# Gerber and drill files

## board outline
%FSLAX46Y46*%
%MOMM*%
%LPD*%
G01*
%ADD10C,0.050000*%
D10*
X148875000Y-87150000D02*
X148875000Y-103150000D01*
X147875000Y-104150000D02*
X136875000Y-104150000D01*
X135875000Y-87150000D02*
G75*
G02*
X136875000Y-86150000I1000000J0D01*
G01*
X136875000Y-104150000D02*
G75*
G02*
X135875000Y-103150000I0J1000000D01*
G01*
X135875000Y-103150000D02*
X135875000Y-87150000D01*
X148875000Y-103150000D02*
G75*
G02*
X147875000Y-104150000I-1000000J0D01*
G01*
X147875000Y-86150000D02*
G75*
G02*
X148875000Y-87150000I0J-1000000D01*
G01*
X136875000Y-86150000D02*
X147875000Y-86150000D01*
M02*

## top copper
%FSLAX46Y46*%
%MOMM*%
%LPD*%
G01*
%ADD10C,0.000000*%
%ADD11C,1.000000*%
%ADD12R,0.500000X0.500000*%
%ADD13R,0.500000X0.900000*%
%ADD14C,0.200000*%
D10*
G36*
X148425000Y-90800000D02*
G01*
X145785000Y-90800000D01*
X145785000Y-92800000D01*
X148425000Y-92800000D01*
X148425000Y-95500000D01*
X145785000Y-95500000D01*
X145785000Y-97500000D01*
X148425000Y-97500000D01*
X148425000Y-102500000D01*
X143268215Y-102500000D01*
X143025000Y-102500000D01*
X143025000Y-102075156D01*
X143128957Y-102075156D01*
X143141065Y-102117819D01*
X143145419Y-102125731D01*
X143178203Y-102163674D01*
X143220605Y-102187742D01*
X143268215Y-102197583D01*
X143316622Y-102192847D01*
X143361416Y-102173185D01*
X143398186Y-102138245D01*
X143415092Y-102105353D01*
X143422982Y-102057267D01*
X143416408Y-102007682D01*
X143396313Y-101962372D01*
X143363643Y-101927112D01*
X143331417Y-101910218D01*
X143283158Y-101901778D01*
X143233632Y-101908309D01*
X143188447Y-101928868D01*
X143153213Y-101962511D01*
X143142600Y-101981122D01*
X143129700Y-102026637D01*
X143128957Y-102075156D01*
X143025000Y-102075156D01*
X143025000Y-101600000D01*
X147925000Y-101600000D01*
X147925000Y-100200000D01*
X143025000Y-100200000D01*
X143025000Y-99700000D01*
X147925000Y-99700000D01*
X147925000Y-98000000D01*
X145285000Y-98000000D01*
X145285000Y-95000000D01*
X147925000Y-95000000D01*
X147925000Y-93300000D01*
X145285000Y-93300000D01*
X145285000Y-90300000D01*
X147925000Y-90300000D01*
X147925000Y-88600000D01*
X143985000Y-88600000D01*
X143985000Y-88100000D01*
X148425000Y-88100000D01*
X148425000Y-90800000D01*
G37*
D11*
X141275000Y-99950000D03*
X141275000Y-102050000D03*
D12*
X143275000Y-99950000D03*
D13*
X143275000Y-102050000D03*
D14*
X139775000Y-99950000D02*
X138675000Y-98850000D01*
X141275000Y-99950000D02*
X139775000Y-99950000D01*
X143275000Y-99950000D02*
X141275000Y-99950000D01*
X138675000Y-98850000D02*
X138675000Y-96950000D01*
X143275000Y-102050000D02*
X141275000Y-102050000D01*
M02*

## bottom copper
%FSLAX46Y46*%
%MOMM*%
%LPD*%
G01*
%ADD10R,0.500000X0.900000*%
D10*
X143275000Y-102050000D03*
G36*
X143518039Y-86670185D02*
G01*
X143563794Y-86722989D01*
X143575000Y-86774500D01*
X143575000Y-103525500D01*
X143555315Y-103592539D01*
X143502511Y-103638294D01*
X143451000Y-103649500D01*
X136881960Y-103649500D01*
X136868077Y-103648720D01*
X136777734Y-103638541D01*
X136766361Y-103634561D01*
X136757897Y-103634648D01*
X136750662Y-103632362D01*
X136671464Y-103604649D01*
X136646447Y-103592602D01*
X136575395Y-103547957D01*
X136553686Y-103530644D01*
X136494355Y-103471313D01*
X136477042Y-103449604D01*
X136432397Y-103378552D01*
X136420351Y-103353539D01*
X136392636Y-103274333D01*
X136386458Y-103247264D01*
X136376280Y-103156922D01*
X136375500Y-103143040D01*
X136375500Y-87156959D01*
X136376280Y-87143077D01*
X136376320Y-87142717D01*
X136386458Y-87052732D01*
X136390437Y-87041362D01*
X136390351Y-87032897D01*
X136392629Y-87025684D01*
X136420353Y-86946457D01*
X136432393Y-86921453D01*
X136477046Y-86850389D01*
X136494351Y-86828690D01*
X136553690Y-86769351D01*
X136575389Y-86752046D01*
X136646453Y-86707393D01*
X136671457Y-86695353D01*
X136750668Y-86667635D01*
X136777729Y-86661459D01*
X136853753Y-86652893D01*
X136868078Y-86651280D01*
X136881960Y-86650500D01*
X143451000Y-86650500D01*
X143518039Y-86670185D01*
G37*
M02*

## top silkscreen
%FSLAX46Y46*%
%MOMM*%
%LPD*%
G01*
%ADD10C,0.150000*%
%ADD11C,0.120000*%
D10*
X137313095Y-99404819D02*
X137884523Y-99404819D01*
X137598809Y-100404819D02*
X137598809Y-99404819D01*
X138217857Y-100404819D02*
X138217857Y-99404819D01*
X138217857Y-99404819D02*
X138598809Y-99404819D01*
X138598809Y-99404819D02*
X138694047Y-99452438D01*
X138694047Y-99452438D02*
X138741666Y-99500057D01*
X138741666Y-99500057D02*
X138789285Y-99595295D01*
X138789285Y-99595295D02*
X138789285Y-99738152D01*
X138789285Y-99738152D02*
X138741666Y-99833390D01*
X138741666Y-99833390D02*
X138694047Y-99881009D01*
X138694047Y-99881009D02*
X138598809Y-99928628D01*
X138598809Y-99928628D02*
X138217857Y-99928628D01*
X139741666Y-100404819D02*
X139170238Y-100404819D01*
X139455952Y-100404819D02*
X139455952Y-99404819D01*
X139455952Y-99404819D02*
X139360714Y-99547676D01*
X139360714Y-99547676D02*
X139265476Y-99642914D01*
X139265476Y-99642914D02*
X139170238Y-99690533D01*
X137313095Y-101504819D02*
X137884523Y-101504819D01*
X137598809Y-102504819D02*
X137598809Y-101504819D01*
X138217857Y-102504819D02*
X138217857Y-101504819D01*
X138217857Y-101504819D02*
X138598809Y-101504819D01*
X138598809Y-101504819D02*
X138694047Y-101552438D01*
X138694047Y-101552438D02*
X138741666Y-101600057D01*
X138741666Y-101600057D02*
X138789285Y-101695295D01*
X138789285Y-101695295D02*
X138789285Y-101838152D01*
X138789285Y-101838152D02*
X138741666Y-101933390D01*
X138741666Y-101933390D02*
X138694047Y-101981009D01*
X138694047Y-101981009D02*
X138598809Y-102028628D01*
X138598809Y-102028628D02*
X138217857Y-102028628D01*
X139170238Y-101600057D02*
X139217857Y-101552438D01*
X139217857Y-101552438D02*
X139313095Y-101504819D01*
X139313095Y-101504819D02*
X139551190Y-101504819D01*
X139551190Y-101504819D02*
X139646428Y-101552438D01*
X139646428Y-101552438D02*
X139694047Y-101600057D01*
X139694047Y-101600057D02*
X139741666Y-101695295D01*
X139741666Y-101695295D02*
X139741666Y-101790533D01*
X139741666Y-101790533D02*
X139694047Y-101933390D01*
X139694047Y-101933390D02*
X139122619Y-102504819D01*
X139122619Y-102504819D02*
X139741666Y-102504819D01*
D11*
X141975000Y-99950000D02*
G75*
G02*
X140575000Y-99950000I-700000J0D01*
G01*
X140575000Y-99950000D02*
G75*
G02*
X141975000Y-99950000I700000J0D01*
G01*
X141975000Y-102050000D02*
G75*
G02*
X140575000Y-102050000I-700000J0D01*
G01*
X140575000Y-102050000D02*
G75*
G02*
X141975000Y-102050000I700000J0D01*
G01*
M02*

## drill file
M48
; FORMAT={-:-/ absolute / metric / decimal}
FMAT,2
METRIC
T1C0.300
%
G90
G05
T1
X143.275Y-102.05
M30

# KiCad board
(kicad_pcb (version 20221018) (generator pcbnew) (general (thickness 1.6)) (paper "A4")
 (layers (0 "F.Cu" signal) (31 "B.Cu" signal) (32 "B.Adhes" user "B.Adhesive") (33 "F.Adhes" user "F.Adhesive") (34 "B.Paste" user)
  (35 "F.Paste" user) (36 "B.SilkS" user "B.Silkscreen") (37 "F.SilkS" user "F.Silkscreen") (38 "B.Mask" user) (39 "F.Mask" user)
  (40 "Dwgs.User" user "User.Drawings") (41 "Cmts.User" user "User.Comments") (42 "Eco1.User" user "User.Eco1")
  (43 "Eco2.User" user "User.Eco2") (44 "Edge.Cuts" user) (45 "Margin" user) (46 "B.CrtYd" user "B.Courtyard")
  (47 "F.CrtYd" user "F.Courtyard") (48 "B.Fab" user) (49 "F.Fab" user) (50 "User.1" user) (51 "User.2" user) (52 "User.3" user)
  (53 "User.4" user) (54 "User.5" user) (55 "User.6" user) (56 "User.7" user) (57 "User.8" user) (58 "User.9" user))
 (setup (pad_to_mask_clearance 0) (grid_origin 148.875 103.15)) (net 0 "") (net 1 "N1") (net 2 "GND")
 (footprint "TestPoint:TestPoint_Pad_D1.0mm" (layer "F.Cu") (at 141.275 99.95)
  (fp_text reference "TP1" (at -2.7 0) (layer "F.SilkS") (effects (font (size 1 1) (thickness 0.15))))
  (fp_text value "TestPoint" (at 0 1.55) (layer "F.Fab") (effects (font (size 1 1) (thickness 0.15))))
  (fp_circle (center 0 0) (end 0 0.7) (stroke (width 0.12) (type solid)) (fill none) (layer "F.SilkS"))
  (pad "1" smd circle (at 0 0) (size 1 1) (layers "F.Cu" "F.Mask") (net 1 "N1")))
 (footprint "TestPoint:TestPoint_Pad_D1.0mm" (layer "F.Cu") (at 141.275 102.05)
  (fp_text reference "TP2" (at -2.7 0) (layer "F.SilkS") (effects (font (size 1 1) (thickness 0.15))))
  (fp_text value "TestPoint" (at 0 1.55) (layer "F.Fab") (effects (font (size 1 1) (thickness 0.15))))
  (fp_circle (center 0 0) (end 0 0.7) (stroke (width 0.12) (type solid)) (fill none) (layer "F.SilkS"))
  (pad "1" smd circle (at 0 0) (size 1 1) (layers "F.Cu" "F.Mask") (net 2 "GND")))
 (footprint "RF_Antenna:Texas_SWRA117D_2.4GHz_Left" (layer "F.Cu") (at 143.275 99.95 -90) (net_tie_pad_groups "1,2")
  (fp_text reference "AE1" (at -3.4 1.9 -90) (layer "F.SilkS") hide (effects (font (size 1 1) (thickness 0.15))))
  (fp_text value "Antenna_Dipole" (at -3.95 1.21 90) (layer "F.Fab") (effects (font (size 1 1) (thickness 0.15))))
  (fp_poly
   (pts (xy -2.45 -2.51) (xy -4.45 -2.51) (xy -4.45 -5.15) (xy -7.15 -5.15) (xy -7.15 -2.51) (xy -9.15 -2.51) (xy -9.15 -5.15)
    (xy -11.85 -5.15) (xy -11.85 -0.71) (xy -11.35 -0.71) (xy -11.35 -4.65) (xy -9.65 -4.65) (xy -9.65 -2.01) (xy -6.65 -2.01)
    (xy -6.65 -4.65) (xy -4.95 -4.65) (xy -4.95 -2.01) (xy -1.95 -2.01) (xy -1.95 -4.65) (xy -0.25 -4.65) (xy -0.25 0.25) (xy 0.25 0.25)
    (xy 0.25 -4.65) (xy 1.65 -4.65) (xy 1.65 0.25) (xy 2.55 0.25) (xy 2.55 0.006785) (xy 2.247583 0.006785) (xy 2.237742 0.054395)
    (xy 2.213674 0.096797) (xy 2.175731 0.129581) (xy 2.167819 0.133935) (xy 2.125156 0.146043) (xy 2.076637 0.1453) (xy 2.031122 0.1324)
    (xy 2.012511 0.121787) (xy 1.978868 0.086553) (xy 1.958309 0.041368) (xy 1.951778 -0.008158) (xy 1.960218 -0.056417)
    (xy 1.977112 -0.088643) (xy 2.012372 -0.121313) (xy 2.057682 -0.141408) (xy 2.107267 -0.147982) (xy 2.155353 -0.140092)
    (xy 2.188245 -0.123186) (xy 2.223185 -0.086416) (xy 2.242847 -0.041622) (xy 2.247583 0.006785) (xy 2.55 0.006785) (xy 2.55 -5.15)
    (xy -2.45 -5.15) (xy -2.45 -2.51))
   (stroke (width 0) (type solid)) (fill solid) (layer "F.Cu"))
  (pad "1" connect rect (at 0 0 270) (size 0.5 0.5) (layers "F.Cu") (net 1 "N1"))
  (pad "2" thru_hole rect (at 2.1 0 270) (size 0.9 0.5) (drill 0.3) (layers "*.Cu") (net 2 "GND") (zone_connect 2)))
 (gr_line (start 148.875 87.15) (end 148.875 103.15) (stroke (width 0.05) (type default)) (layer "Edge.Cuts"))
 (gr_line (start 147.875 104.15) (end 136.875 104.15) (stroke (width 0.05) (type default)) (layer "Edge.Cuts"))
 (gr_arc (start 135.875 87.15) (mid 136.167893 86.442893) (end 136.875 86.15) (stroke (width 0.05) (type default)) (layer "Edge.Cuts"))
 (gr_arc (start 136.875 104.15) (mid 136.167893 103.857107) (end 135.875 103.15) (stroke (width 0.05) (type default)) (layer "Edge.Cuts"))
 (gr_line (start 135.875 103.15) (end 135.875 87.15) (stroke (width 0.05) (type default)) (layer "Edge.Cuts"))
 (gr_arc (start 148.875 103.15) (mid 148.582107 103.857107) (end 147.875 104.15) (stroke (width 0.05) (type default)) (layer "Edge.Cuts"))
 (gr_arc (start 147.875 86.15) (mid 148.582107 86.442893) (end 148.875 87.15) (stroke (width 0.05) (type default)) (layer "Edge.Cuts"))
 (gr_line (start 136.875 86.15) (end 147.875 86.15) (stroke (width 0.05) (type default)) (layer "Edge.Cuts"))
 (segment (start 139.775 99.95) (end 138.675 98.85) (width 0.2) (layer "F.Cu") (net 1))
 (segment (start 141.275 99.95) (end 139.775 99.95) (width 0.2) (layer "F.Cu") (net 1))
 (segment (start 143.275 99.95) (end 141.275 99.95) (width 0.2) (layer "F.Cu") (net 1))
 (segment (start 138.675 98.85) (end 138.675 96.95) (width 0.2) (layer "F.Cu") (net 1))
 (segment (start 143.275 102.05) (end 141.275 102.05) (width 0.2) (layer "F.Cu") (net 2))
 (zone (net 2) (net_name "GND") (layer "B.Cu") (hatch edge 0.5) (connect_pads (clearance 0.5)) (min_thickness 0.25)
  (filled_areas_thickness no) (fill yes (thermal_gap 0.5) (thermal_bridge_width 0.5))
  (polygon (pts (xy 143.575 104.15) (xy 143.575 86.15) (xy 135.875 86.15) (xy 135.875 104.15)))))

